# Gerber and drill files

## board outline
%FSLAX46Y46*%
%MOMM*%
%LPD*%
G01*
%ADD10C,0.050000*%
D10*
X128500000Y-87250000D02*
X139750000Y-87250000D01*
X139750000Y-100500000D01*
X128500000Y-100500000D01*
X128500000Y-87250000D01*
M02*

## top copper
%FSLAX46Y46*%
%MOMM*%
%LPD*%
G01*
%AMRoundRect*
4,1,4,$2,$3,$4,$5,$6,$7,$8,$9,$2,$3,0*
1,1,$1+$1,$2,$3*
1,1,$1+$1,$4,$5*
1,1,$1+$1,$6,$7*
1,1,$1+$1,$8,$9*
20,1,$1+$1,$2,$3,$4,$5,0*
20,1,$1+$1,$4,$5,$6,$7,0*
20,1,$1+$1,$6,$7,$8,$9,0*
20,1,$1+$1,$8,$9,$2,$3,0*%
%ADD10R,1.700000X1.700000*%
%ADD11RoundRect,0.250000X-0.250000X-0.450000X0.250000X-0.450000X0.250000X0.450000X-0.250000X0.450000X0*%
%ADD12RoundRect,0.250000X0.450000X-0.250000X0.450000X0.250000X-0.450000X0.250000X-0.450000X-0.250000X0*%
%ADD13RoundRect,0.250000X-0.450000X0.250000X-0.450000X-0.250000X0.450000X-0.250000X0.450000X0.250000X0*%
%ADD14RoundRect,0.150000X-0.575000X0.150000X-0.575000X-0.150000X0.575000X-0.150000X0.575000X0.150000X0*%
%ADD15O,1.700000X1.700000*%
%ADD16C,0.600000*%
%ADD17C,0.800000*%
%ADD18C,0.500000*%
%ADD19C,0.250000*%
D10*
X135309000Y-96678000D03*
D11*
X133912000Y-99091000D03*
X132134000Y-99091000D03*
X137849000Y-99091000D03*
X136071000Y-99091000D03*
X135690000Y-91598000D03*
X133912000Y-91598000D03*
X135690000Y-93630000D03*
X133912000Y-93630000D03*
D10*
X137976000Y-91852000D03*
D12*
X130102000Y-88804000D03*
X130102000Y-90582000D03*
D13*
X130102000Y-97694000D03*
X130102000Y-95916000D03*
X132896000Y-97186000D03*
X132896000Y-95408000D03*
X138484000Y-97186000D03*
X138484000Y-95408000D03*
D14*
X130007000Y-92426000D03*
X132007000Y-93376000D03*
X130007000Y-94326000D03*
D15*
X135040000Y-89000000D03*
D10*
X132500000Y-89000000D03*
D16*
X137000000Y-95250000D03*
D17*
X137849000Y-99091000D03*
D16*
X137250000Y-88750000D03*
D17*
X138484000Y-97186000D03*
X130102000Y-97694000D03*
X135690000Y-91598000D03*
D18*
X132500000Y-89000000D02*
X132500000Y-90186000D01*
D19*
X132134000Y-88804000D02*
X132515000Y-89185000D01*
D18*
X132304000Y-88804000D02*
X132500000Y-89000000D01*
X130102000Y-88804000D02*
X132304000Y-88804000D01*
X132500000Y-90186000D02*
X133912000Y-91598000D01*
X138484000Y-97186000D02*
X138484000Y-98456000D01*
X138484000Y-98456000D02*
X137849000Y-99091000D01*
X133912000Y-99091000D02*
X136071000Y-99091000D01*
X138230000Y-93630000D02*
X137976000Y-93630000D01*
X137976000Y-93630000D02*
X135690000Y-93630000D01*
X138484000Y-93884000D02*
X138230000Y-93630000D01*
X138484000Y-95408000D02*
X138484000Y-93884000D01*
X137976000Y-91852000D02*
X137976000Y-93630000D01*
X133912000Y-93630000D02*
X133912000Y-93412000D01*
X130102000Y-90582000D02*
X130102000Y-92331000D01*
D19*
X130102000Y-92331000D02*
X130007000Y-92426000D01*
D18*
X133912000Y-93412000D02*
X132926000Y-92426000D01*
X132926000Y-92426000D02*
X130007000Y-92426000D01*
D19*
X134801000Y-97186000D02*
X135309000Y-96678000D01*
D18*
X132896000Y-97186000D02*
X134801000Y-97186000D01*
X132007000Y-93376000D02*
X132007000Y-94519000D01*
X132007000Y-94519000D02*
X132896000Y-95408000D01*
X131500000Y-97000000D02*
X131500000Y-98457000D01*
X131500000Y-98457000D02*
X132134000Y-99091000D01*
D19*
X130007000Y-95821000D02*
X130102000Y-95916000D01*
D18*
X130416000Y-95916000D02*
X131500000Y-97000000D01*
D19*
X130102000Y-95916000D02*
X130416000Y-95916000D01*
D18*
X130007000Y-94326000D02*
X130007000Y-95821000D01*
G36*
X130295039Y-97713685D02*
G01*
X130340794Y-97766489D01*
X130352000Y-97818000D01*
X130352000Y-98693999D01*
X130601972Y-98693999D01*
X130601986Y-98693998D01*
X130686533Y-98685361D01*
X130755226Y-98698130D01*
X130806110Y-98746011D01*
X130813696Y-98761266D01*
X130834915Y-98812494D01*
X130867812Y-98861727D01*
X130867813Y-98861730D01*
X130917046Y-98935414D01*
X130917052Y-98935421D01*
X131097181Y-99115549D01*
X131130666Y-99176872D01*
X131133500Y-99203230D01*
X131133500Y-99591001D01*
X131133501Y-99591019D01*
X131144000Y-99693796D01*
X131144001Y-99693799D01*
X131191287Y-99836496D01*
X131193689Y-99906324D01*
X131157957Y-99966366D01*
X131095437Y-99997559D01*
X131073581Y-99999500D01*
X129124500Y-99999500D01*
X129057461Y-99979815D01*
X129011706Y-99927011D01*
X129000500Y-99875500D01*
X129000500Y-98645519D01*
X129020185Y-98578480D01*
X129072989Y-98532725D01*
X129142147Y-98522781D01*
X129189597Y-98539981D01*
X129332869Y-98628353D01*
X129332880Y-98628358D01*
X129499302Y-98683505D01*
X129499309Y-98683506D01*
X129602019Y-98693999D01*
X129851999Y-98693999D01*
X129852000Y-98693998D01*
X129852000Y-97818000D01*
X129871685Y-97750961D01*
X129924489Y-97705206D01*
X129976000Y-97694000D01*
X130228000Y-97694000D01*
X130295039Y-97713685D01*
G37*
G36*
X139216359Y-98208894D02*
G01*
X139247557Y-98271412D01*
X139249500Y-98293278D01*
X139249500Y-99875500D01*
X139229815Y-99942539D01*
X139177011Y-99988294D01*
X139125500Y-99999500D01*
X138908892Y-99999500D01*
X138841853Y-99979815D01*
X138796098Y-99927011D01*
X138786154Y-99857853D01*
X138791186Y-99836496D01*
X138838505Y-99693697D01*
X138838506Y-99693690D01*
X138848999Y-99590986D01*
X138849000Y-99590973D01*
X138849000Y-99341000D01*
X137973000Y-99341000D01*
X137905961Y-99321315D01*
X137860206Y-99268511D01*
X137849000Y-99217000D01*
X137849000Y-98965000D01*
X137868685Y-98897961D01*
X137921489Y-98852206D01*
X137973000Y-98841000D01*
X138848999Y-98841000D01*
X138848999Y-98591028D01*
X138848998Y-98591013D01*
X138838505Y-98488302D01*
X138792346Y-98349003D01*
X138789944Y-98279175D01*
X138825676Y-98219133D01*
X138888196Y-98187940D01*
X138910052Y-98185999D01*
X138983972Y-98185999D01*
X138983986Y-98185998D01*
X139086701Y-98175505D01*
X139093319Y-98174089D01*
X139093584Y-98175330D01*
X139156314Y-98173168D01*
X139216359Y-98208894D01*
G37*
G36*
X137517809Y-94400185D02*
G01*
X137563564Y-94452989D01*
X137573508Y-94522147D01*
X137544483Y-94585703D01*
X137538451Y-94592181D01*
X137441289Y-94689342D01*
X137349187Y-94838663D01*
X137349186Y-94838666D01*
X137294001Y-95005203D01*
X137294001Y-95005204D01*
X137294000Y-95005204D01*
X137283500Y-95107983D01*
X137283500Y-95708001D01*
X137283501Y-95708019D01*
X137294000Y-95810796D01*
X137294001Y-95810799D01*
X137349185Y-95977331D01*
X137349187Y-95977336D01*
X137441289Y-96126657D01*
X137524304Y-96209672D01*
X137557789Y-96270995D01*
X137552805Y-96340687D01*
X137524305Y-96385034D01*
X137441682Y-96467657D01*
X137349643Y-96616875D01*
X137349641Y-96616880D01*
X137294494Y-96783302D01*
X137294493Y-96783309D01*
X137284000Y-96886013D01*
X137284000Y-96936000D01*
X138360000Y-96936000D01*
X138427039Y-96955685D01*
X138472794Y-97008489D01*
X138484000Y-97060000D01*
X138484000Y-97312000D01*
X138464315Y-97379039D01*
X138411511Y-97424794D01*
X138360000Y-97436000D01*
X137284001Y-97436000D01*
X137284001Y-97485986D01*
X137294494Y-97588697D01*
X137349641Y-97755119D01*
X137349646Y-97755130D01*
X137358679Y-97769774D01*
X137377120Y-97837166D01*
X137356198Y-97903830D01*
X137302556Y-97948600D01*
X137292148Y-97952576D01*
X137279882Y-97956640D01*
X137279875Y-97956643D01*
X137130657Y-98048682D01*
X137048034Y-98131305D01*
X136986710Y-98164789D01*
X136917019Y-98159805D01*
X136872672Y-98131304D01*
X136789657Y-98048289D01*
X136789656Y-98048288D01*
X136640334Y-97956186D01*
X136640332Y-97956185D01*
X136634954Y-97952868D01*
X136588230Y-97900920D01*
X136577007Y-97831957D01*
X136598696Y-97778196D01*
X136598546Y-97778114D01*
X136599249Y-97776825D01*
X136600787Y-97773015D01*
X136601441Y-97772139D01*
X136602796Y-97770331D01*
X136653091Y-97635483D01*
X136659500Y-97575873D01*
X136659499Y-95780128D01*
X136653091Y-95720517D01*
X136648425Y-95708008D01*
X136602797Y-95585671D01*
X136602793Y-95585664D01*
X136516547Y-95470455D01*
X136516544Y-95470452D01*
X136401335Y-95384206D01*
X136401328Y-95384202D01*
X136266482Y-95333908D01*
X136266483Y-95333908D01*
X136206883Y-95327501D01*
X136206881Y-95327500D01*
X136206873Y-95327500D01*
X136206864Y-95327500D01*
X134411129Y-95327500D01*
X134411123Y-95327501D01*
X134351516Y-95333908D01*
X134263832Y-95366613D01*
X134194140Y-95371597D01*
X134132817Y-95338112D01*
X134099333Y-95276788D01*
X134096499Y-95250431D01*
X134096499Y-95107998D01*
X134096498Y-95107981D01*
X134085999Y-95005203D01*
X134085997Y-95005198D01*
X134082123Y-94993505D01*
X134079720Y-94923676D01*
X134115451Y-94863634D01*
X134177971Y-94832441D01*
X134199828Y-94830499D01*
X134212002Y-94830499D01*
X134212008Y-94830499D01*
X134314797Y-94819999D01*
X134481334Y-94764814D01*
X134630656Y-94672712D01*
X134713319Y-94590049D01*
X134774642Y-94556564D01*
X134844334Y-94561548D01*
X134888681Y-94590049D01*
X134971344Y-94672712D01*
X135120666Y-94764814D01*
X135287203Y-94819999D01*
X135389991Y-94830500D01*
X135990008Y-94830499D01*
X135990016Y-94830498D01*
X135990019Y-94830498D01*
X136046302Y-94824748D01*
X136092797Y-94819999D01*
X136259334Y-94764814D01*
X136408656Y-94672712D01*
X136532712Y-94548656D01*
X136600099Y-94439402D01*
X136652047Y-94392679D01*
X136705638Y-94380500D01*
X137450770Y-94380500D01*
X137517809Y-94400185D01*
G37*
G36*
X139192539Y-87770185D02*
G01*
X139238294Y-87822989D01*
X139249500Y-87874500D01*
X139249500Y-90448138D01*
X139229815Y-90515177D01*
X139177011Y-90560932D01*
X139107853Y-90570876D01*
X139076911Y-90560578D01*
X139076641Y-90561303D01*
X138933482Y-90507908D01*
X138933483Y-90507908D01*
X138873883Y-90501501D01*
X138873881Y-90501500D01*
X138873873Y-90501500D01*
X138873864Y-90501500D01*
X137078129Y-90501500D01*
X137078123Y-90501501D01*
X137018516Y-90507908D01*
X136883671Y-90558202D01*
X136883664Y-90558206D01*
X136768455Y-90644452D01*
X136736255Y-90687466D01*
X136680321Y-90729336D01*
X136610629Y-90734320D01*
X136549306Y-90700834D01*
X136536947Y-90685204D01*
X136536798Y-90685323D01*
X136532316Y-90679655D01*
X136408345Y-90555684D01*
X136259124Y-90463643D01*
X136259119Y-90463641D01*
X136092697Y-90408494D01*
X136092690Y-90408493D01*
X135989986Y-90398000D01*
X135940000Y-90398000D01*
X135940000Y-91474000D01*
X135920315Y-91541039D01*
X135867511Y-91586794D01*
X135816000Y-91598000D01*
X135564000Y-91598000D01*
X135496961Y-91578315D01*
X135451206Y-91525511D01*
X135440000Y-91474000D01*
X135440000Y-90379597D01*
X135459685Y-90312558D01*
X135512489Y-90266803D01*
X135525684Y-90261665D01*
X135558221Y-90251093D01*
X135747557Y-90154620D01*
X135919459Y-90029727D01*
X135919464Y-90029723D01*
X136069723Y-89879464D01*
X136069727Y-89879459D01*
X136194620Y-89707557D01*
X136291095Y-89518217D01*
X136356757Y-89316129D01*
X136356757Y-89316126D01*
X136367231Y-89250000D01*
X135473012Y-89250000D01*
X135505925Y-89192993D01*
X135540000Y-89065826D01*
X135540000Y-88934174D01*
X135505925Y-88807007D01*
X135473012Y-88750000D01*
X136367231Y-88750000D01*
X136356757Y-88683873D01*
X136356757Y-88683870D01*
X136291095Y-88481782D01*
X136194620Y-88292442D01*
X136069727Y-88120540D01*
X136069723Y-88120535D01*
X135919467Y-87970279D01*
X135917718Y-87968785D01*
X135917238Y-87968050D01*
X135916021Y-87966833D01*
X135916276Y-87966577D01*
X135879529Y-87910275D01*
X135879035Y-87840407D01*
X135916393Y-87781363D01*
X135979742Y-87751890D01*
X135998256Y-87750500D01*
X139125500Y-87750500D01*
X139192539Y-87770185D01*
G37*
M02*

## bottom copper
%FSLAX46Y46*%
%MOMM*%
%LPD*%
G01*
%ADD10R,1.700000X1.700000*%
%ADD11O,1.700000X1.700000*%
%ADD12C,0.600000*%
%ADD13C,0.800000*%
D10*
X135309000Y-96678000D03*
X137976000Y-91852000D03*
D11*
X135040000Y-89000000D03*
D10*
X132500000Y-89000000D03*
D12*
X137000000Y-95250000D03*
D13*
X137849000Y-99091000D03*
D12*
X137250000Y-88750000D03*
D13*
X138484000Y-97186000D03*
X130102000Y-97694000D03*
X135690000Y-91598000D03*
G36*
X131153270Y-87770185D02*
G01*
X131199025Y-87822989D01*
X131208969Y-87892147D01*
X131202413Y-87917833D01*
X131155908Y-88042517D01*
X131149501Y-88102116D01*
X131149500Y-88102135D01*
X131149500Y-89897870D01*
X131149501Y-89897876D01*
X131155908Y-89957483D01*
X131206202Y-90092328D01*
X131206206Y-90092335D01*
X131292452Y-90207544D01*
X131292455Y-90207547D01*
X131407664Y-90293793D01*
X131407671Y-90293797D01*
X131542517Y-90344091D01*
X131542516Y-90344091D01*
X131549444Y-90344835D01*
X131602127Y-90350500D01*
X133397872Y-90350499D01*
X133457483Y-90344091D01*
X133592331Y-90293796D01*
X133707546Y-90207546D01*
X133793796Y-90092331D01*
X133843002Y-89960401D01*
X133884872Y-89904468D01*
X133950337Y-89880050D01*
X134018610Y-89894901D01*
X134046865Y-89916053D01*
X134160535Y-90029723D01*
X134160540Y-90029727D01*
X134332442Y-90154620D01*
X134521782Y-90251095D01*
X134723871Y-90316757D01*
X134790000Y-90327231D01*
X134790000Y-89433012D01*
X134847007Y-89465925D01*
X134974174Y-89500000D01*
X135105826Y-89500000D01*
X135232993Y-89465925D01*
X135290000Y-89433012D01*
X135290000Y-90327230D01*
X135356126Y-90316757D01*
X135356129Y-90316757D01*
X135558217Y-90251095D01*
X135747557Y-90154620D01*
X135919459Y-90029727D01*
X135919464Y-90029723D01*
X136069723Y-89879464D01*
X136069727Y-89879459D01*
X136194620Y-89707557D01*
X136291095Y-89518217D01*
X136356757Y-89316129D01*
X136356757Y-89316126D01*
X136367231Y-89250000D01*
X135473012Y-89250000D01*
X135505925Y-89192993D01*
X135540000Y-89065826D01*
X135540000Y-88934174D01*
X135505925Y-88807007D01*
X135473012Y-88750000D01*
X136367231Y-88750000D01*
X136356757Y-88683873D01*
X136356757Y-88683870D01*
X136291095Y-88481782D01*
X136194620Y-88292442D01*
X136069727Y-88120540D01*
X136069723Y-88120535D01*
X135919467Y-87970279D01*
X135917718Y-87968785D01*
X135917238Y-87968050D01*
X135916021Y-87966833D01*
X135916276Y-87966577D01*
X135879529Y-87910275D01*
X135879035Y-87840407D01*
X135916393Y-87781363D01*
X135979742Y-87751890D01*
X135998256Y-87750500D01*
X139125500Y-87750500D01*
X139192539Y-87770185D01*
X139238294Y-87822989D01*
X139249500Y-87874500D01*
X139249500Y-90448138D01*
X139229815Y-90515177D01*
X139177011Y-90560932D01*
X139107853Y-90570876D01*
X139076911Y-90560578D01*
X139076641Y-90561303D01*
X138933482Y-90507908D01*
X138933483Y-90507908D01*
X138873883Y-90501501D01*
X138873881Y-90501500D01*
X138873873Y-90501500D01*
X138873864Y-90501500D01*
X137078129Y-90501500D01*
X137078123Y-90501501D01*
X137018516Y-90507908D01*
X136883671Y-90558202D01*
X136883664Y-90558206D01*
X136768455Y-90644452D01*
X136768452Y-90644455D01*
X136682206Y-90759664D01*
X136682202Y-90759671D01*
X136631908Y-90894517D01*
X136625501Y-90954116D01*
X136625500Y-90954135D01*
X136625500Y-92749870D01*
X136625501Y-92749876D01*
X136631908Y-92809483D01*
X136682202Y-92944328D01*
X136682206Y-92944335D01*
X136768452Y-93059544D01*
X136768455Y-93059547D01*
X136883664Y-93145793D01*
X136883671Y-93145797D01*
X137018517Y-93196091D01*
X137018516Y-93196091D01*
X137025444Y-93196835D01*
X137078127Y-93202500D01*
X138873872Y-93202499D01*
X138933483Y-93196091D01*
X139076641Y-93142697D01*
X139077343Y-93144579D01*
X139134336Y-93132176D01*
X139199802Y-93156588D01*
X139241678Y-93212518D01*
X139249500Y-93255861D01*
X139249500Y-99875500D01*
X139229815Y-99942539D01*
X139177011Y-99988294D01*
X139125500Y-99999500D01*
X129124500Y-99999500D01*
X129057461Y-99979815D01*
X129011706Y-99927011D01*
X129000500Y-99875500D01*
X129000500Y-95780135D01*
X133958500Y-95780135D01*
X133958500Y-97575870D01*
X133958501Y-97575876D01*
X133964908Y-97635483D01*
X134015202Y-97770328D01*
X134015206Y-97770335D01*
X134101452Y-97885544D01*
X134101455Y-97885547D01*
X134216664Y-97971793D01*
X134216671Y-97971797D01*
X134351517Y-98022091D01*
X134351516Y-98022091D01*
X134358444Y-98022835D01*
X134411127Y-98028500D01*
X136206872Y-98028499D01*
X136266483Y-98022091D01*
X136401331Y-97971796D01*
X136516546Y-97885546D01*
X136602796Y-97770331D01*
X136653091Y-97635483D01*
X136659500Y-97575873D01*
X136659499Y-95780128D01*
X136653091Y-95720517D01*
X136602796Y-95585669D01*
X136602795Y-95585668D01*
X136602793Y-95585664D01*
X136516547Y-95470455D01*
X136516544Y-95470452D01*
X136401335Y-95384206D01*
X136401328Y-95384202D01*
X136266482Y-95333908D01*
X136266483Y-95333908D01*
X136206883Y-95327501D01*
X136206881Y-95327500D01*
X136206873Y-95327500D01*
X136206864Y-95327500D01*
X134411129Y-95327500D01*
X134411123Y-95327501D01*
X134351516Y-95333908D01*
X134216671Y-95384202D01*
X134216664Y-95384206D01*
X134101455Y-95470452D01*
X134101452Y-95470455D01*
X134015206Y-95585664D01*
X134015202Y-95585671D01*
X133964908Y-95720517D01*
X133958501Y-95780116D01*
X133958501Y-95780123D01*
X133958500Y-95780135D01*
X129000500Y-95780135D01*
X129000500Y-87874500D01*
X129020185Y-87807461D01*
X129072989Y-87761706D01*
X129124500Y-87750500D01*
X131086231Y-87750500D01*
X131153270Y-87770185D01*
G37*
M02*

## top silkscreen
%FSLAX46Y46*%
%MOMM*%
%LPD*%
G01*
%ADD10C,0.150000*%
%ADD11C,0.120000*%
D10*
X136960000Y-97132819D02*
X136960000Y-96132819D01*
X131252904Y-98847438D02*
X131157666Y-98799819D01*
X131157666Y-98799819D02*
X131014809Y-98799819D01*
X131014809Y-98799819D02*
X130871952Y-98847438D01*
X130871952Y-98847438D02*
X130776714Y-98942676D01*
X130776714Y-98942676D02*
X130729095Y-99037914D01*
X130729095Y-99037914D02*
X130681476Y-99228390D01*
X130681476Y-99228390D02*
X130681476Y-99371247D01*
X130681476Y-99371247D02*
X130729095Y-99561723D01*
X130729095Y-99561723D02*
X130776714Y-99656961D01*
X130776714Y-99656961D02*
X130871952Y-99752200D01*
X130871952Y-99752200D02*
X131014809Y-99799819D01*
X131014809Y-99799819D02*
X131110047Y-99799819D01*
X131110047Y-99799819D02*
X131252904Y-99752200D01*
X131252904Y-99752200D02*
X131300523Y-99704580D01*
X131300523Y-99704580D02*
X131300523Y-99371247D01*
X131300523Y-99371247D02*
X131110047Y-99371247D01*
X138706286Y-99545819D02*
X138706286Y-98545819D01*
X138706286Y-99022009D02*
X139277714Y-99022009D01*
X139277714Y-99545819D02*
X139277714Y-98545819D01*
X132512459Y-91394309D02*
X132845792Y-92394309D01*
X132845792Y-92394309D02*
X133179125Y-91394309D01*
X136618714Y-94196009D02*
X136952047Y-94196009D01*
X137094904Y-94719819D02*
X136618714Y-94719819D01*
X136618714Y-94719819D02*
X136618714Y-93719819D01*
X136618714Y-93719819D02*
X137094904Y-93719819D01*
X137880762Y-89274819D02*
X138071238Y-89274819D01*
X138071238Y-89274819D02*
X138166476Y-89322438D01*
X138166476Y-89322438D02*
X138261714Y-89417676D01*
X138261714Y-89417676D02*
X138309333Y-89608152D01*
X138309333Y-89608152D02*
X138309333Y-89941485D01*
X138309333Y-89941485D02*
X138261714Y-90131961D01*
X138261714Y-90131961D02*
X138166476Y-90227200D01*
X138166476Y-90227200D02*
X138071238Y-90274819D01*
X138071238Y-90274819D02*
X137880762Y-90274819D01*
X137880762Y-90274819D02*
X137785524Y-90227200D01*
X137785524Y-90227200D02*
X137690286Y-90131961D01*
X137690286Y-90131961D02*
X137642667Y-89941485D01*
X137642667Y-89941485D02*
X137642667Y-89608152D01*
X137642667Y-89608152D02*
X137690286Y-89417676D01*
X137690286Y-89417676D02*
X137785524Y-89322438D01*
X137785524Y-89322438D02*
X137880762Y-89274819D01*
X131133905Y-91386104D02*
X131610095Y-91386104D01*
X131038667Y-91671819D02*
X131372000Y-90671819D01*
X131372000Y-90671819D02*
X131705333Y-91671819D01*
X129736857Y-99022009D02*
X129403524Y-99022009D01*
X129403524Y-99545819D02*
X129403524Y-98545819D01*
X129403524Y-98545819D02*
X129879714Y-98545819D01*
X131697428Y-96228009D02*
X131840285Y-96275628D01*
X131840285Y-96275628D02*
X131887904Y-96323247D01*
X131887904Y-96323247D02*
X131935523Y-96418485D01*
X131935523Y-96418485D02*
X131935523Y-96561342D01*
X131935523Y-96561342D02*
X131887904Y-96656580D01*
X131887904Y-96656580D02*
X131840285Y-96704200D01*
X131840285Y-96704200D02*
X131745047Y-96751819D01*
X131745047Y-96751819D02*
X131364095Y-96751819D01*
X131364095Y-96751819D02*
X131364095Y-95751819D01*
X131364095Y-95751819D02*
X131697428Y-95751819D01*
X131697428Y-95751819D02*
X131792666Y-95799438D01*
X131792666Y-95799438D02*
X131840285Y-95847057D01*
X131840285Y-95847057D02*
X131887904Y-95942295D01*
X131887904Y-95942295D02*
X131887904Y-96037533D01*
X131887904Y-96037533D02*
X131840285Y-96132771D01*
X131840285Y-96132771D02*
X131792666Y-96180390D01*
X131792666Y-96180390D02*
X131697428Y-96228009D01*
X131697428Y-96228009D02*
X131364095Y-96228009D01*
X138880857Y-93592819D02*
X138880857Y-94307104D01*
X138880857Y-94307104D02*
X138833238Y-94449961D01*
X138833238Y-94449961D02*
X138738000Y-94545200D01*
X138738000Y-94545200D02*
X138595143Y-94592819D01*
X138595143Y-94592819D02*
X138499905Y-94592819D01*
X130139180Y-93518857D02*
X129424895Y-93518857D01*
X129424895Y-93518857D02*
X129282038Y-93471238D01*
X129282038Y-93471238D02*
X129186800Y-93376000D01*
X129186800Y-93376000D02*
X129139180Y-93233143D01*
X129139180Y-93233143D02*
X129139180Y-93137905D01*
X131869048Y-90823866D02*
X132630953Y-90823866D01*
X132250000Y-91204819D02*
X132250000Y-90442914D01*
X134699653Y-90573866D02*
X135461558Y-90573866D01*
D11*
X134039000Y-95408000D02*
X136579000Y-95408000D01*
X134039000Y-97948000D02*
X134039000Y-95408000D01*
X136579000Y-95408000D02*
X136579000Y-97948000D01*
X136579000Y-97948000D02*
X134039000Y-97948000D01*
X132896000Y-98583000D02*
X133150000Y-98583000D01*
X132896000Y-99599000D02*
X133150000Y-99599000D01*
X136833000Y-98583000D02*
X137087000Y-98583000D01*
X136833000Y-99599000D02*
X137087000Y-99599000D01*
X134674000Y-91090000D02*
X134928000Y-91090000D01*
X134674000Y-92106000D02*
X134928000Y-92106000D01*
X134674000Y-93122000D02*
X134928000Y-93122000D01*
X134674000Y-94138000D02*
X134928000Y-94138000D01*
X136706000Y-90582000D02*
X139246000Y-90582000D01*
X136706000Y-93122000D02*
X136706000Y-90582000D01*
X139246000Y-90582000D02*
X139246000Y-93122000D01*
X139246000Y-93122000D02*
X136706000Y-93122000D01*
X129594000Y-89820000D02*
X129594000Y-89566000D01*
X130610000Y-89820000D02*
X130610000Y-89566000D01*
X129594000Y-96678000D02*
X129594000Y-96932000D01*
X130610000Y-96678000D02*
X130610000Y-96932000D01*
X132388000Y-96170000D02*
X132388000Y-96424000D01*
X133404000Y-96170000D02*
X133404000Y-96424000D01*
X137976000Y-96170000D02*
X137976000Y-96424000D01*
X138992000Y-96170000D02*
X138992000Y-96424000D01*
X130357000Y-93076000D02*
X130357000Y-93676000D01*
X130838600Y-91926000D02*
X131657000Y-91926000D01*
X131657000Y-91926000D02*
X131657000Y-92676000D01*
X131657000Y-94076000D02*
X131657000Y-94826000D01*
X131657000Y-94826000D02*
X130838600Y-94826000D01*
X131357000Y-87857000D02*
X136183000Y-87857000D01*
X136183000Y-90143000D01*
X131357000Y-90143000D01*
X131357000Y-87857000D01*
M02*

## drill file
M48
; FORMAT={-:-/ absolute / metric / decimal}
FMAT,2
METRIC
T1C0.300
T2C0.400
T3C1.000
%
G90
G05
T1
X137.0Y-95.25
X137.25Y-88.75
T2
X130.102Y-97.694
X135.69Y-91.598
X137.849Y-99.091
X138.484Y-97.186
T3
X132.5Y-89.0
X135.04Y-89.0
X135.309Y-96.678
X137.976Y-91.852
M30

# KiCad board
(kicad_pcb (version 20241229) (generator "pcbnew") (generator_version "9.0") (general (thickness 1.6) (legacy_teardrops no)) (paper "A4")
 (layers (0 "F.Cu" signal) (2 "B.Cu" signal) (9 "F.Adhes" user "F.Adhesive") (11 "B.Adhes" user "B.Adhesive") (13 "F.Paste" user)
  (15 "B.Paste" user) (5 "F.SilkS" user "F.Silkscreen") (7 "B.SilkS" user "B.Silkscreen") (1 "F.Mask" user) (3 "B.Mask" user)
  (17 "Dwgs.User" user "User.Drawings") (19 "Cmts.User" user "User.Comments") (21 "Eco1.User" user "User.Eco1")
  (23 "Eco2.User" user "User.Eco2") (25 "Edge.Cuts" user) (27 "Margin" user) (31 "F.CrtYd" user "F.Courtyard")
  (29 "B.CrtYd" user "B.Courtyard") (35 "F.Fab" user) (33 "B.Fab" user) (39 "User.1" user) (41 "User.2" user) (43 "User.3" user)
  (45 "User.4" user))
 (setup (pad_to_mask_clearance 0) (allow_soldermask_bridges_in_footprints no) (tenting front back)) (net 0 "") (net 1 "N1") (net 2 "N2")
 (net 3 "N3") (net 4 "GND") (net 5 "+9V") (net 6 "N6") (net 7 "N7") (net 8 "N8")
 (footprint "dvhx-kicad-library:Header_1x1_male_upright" (layer "F.Cu") (at 135.309 96.678)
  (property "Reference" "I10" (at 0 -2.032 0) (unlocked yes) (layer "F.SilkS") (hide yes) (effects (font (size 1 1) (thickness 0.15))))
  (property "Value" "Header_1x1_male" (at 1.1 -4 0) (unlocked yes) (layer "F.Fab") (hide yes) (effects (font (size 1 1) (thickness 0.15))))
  (fp_line (start -1.27 -1.27) (end 1.27 -1.27) (stroke (width 0.12) (type solid)) (layer "F.SilkS"))
  (fp_line (start -1.27 1.27) (end -1.27 -1.27) (stroke (width 0.12) (type solid)) (layer "F.SilkS"))
  (fp_line (start 1.27 -1.27) (end 1.27 1.27) (stroke (width 0.12) (type solid)) (layer "F.SilkS"))
  (fp_line (start 1.27 1.27) (end -1.27 1.27) (stroke (width 0.12) (type solid)) (layer "F.SilkS"))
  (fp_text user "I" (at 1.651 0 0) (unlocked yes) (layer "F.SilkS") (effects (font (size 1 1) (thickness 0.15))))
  (pad "1" thru_hole rect (at 0 0) (size 1.7 1.7) (drill 1) (layers "*.Cu" "*.Mask") (remove_unused_layers no) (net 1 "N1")))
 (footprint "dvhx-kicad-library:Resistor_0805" (layer "F.Cu") (at 133.023 99.091)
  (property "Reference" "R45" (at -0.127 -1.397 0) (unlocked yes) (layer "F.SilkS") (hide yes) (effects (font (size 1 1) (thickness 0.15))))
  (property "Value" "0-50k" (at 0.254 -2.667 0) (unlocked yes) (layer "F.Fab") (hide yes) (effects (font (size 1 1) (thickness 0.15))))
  (fp_line (start -0.127 -0.508) (end 0.127 -0.508) (stroke (width 0.12) (type solid)) (layer "F.SilkS"))
  (fp_line (start -0.127 0.508) (end 0.127 0.508) (stroke (width 0.12) (type solid)) (layer "F.SilkS"))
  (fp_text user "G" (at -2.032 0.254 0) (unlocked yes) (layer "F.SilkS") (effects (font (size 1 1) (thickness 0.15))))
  (pad "1" smd roundrect (at 0.889 0) (size 1 1.4) (layers "F.Cu" "F.Mask" "F.Paste") (roundrect_rratio 0.25) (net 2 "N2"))
  (pad "2" smd roundrect (at -0.889 0) (size 1 1.4) (layers "F.Cu" "F.Mask" "F.Paste") (roundrect_rratio 0.25) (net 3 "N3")))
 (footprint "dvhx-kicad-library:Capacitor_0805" (layer "F.Cu") (at 136.96 99.091)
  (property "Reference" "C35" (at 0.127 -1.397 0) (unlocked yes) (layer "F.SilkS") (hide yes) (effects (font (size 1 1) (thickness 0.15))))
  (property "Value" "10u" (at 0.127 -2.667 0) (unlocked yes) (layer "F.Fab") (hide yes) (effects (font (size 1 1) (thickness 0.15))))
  (fp_line (start -0.127 -0.508) (end 0.127 -0.508) (stroke (width 0.12) (type solid)) (layer "F.SilkS"))
  (fp_line (start -0.127 0.508) (end 0.127 0.508) (stroke (width 0.12) (type solid)) (layer "F.SilkS"))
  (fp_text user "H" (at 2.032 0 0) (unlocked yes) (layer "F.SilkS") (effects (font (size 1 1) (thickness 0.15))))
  (pad "1" smd roundrect (at 0.889 0) (size 1 1.4) (layers "F.Cu" "F.Mask" "F.Paste") (roundrect_rratio 0.25) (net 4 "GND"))
  (pad "2" smd roundrect (at -0.889 0) (size 1 1.4) (layers "F.Cu" "F.Mask" "F.Paste") (roundrect_rratio 0.25) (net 2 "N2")))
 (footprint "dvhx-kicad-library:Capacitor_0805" (layer "F.Cu") (at 134.801 91.598)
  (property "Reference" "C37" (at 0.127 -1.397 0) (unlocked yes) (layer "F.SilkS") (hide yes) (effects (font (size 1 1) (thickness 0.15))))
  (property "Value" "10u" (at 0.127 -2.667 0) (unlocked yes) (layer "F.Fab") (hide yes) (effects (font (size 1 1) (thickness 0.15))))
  (fp_line (start -0.127 -0.508) (end 0.127 -0.508) (stroke (width 0.12) (type solid)) (layer "F.SilkS"))
  (fp_line (start -0.127 0.508) (end 0.127 0.508) (stroke (width 0.12) (type solid)) (layer "F.SilkS"))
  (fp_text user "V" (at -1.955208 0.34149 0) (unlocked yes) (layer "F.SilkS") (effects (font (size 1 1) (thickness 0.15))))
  (pad "1" smd roundrect (at 0.889 0) (size 1 1.4) (layers "F.Cu" "F.Mask" "F.Paste") (roundrect_rratio 0.25) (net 4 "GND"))
  (pad "2" smd roundrect (at -0.889 0) (size 1 1.4) (layers "F.Cu" "F.Mask" "F.Paste") (roundrect_rratio 0.25) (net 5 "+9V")))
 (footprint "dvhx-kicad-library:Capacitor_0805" (layer "F.Cu") (at 134.801 93.63)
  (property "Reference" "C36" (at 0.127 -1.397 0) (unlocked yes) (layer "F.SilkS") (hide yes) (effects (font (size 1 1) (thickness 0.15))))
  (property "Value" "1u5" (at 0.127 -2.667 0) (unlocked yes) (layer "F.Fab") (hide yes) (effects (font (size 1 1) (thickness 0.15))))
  (fp_line (start -0.127 -0.508) (end 0.127 -0.508) (stroke (width 0.12) (type solid)) (layer "F.SilkS"))
  (fp_line (start -0.127 0.508) (end 0.127 0.508) (stroke (width 0.12) (type solid)) (layer "F.SilkS"))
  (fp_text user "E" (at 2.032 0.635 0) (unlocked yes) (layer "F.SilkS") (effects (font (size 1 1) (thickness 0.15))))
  (pad "1" smd roundrect (at 0.889 0) (size 1 1.4) (layers "F.Cu" "F.Mask" "F.Paste") (roundrect_rratio 0.25) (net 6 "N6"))
  (pad "2" smd roundrect (at -0.889 0) (size 1 1.4) (layers "F.Cu" "F.Mask" "F.Paste") (roundrect_rratio 0.25) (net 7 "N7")))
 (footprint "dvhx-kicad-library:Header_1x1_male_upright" (layer "F.Cu") (at 137.976 91.852)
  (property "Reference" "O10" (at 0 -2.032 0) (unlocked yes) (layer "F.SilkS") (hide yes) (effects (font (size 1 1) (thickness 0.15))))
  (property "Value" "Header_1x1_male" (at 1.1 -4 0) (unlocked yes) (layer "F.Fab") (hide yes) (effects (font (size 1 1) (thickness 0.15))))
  (fp_line (start -1.27 -1.27) (end 1.27 -1.27) (stroke (width 0.12) (type solid)) (layer "F.SilkS"))
  (fp_line (start -1.27 1.27) (end -1.27 -1.27) (stroke (width 0.12) (type solid)) (layer "F.SilkS"))
  (fp_line (start 1.27 -1.27) (end 1.27 1.27) (stroke (width 0.12) (type solid)) (layer "F.SilkS"))
  (fp_line (start 1.27 1.27) (end -1.27 1.27) (stroke (width 0.12) (type solid)) (layer "F.SilkS"))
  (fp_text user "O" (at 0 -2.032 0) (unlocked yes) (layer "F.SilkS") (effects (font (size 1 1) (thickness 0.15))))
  (pad "1" thru_hole rect (at 0 0) (size 1.7 1.7) (drill 1) (layers "*.Cu" "*.Mask") (remove_unused_layers no) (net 6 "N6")))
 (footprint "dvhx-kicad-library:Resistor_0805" (layer "F.Cu") (at 130.102 89.693 90)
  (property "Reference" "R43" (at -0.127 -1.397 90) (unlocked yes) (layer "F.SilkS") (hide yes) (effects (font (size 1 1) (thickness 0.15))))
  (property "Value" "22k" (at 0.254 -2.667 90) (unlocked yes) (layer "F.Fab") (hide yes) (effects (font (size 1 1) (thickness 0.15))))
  (fp_line (start -0.127 -0.508) (end 0.127 -0.508) (stroke (width 0.12) (type solid)) (layer "F.SilkS"))
  (fp_line (start -0.127 0.508) (end 0.127 0.508) (stroke (width 0.12) (type solid)) (layer "F.SilkS"))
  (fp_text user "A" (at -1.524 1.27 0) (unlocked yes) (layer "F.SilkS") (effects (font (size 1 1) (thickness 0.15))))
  (pad "1" smd roundrect (at 0.889 0 90) (size 1 1.4) (layers "F.Cu" "F.Mask" "F.Paste") (roundrect_rratio 0.25) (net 5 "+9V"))
  (pad "2" smd roundrect (at -0.889 0 90) (size 1 1.4) (layers "F.Cu" "F.Mask" "F.Paste") (roundrect_rratio 0.25) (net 7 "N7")))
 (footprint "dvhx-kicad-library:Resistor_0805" (layer "F.Cu") (at 130.102 96.805 -90)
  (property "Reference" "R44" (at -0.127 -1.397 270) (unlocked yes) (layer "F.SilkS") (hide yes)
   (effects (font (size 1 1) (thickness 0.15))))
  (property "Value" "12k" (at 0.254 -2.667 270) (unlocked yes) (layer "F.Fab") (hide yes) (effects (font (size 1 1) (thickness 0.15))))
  (fp_line (start -0.127 0.508) (end 0.127 0.508) (stroke (width 0.12) (type solid)) (layer "F.SilkS"))
  (fp_line (start -0.127 -0.508) (end 0.127 -0.508) (stroke (width 0.12) (type solid)) (layer "F.SilkS"))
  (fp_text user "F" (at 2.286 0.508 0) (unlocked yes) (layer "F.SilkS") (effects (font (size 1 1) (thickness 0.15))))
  (pad "1" smd roundrect (at 0.889 0 270) (size 1 1.4) (layers "F.Cu" "F.Mask" "F.Paste") (roundrect_rratio 0.25) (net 4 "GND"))
  (pad "2" smd roundrect (at -0.889 0 270) (size 1 1.4) (layers "F.Cu" "F.Mask" "F.Paste") (roundrect_rratio 0.25) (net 3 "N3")))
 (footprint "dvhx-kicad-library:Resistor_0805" (layer "F.Cu") (at 132.896 96.297 -90)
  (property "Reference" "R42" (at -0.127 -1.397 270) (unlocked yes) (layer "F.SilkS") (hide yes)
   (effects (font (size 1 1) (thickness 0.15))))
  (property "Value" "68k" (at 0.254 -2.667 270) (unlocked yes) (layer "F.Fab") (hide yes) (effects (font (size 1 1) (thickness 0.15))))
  (fp_line (start -0.127 0.508) (end 0.127 0.508) (stroke (width 0.12) (type solid)) (layer "F.SilkS"))
  (fp_line (start -0.127 -0.508) (end 0.127 -0.508) (stroke (width 0.12) (type solid)) (layer "F.SilkS"))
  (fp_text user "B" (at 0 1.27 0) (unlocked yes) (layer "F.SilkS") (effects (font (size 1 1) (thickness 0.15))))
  (pad "1" smd roundrect (at 0.889 0 270) (size 1 1.4) (layers "F.Cu" "F.Mask" "F.Paste") (roundrect_rratio 0.25) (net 1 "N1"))
  (pad "2" smd roundrect (at -0.889 0 270) (size 1 1.4) (layers "F.Cu" "F.Mask" "F.Paste") (roundrect_rratio 0.25) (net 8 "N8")))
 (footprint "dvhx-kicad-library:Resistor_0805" (layer "F.Cu") (at 138.484 96.297 -90)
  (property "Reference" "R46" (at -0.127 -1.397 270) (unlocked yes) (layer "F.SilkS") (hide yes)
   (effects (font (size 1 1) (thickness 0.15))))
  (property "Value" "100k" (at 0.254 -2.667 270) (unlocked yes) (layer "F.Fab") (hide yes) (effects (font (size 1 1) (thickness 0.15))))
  (fp_line (start -0.127 0.508) (end 0.127 0.508) (stroke (width 0.12) (type solid)) (layer "F.SilkS"))
  (fp_line (start -0.127 -0.508) (end 0.127 -0.508) (stroke (width 0.12) (type solid)) (layer "F.SilkS"))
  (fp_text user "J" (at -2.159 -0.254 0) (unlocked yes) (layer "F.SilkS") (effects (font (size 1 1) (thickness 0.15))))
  (pad "1" smd roundrect (at 0.889 0 270) (size 1 1.4) (layers "F.Cu" "F.Mask" "F.Paste") (roundrect_rratio 0.25) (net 4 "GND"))
  (pad "2" smd roundrect (at -0.889 0 270) (size 1 1.4) (layers "F.Cu" "F.Mask" "F.Paste") (roundrect_rratio 0.25) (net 6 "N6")))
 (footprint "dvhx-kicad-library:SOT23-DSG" (layer "F.Cu") (at 130.991 93.376 -90)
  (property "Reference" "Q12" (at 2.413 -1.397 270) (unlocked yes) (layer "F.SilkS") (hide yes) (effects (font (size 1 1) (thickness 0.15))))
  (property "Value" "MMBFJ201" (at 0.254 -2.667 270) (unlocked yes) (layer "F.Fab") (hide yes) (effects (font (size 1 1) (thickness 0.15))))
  (fp_line (start -0.3 0.634) (end 0.3 0.634) (stroke (width 0.12) (type solid)) (layer "F.SilkS"))
  (fp_line (start -1.45 0.1524) (end -1.45 -0.666) (stroke (width 0.12) (type solid)) (layer "F.SilkS"))
  (fp_line (start -1.45 -0.666) (end -0.7 -0.666) (stroke (width 0.12) (type solid)) (layer "F.SilkS"))
  (fp_line (start 0.7 -0.666) (end 1.45 -0.666) (stroke (width 0.12) (type solid)) (layer "F.SilkS"))
  (fp_line (start 1.45 -0.666) (end 1.45 0.1524) (stroke (width 0.12) (type solid)) (layer "F.SilkS"))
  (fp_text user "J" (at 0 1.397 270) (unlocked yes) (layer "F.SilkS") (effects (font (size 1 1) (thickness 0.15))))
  (pad "D" smd roundrect (at -0.95 0.984 270) (size 0.6 1.45) (layers "F.Cu" "F.Mask" "F.Paste") (roundrect_rratio 0.25) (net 7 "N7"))
  (pad "G" smd roundrect (at 0 -1.016 270) (size 0.6 1.45) (layers "F.Cu" "F.Mask" "F.Paste") (roundrect_rratio 0.25) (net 8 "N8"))
  (pad "S" smd roundrect (at 0.95 0.984 270) (size 0.6 1.45) (layers "F.Cu" "F.Mask" "F.Paste") (roundrect_rratio 0.25) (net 3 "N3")))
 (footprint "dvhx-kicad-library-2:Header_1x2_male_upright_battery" (layer "F.Cu") (at 132.5 89)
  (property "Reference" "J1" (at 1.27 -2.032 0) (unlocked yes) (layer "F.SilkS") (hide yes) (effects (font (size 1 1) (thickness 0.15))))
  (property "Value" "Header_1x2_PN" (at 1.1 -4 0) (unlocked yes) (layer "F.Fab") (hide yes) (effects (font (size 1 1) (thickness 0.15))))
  (fp_rect (start -1.143 -1.143) (end 3.683 1.143) (stroke (width 0.12) (type solid)) (fill no) (layer "F.SilkS"))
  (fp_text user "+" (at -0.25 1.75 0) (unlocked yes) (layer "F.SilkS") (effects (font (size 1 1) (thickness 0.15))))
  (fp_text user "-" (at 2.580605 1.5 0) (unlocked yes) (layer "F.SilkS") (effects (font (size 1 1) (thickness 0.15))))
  (pad "N" thru_hole oval (at 2.54 0 90) (size 1.7 1.7) (drill 1) (layers "*.Cu" "*.Mask") (remove_unused_layers no) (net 4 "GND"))
  (pad "P" thru_hole rect (at 0 0 90) (size 1.7 1.7) (drill 1) (layers "*.Cu" "*.Mask") (remove_unused_layers no) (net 5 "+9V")))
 (gr_rect (start 128.5 87.25) (end 139.75 100.5) (stroke (width 0.05) (type default)) (fill no) (layer "Edge.Cuts"))
 (segment (start 132.5 89) (end 132.5 90.186) (width 0.5) (layer "F.Cu") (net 5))
 (segment (start 132.134 88.804) (end 132.515 89.185) (width 0.25) (layer "F.Cu") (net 5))
 (segment (start 132.304 88.804) (end 132.5 89) (width 0.5) (layer "F.Cu") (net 5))
 (segment (start 130.102 88.804) (end 132.304 88.804) (width 0.5) (layer "F.Cu") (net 5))
 (segment (start 132.5 90.186) (end 133.912 91.598) (width 0.5) (layer "F.Cu") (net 5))
 (segment (start 138.484 97.186) (end 138.484 98.456) (width 0.5) (layer "F.Cu") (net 4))
 (segment (start 138.484 98.456) (end 137.849 99.091) (width 0.5) (layer "F.Cu") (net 4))
 (via (at 137 95.25) (size 0.6) (drill 0.3) (layers "F.Cu" "B.Cu") (free yes) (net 4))
 (via (at 137.849 99.091) (size 0.8) (drill 0.4) (layers "F.Cu" "B.Cu") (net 4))
 (via (at 137.25 88.75) (size 0.6) (drill 0.3) (layers "F.Cu" "B.Cu") (free yes) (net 4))
 (via (at 138.484 97.186) (size 0.8) (drill 0.4) (layers "F.Cu" "B.Cu") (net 4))
 (via (at 130.102 97.694) (size 0.8) (drill 0.4) (layers "F.Cu" "B.Cu") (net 4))
 (via (at 135.69 91.598) (size 0.8) (drill 0.4) (layers "F.Cu" "B.Cu") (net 4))
 (segment (start 133.912 99.091) (end 136.071 99.091) (width 0.5) (layer "F.Cu") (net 2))
 (segment (start 138.23 93.63) (end 137.976 93.63) (width 0.5) (layer "F.Cu") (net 6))
 (segment (start 137.976 93.63) (end 135.69 93.63) (width 0.5) (layer "F.Cu") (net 6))
 (segment (start 138.484 93.884) (end 138.23 93.63) (width 0.5) (layer "F.Cu") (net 6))
 (segment (start 138.484 95.408) (end 138.484 93.884) (width 0.5) (layer "F.Cu") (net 6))
 (segment (start 137.976 91.852) (end 137.976 93.63) (width 0.5) (layer "F.Cu") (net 6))
 (segment (start 133.912 93.63) (end 133.912 93.412) (width 0.5) (layer "F.Cu") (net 7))
 (segment (start 130.102 90.582) (end 130.102 92.331) (width 0.5) (layer "F.Cu") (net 7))
 (segment (start 130.102 92.331) (end 130.007 92.426) (width 0.25) (layer "F.Cu") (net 7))
 (segment (start 133.912 93.412) (end 132.926 92.426) (width 0.5) (layer "F.Cu") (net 7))
 (segment (start 132.926 92.426) (end 130.007 92.426) (width 0.5) (layer "F.Cu") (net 7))
 (segment (start 134.801 97.186) (end 135.309 96.678) (width 0.25) (layer "F.Cu") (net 1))
 (segment (start 132.896 97.186) (end 134.801 97.186) (width 0.5) (layer "F.Cu") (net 1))
 (segment (start 132.007 93.376) (end 132.007 94.519) (width 0.5) (layer "F.Cu") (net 8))
 (segment (start 132.007 94.519) (end 132.896 95.408) (width 0.5) (layer "F.Cu") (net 8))
 (segment (start 131.5 97) (end 131.5 98.457) (width 0.5) (layer "F.Cu") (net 3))
 (segment (start 131.5 98.457) (end 132.134 99.091) (width 0.5) (layer "F.Cu") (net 3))
 (segment (start 130.007 95.821) (end 130.102 95.916) (width 0.25) (layer "F.Cu") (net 3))
 (segment (start 130.416 95.916) (end 131.5 97) (width 0.5) (layer "F.Cu") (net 3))
 (segment (start 130.102 95.916) (end 130.416 95.916) (width 0.25) (layer "F.Cu") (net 3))
 (segment (start 130.007 94.326) (end 130.007 95.821) (width 0.5) (layer "F.Cu") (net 3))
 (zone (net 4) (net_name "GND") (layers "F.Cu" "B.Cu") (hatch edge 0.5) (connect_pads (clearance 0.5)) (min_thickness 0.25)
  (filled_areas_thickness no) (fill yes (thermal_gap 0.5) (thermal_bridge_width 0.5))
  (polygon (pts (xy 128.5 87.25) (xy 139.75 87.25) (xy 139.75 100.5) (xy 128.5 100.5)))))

